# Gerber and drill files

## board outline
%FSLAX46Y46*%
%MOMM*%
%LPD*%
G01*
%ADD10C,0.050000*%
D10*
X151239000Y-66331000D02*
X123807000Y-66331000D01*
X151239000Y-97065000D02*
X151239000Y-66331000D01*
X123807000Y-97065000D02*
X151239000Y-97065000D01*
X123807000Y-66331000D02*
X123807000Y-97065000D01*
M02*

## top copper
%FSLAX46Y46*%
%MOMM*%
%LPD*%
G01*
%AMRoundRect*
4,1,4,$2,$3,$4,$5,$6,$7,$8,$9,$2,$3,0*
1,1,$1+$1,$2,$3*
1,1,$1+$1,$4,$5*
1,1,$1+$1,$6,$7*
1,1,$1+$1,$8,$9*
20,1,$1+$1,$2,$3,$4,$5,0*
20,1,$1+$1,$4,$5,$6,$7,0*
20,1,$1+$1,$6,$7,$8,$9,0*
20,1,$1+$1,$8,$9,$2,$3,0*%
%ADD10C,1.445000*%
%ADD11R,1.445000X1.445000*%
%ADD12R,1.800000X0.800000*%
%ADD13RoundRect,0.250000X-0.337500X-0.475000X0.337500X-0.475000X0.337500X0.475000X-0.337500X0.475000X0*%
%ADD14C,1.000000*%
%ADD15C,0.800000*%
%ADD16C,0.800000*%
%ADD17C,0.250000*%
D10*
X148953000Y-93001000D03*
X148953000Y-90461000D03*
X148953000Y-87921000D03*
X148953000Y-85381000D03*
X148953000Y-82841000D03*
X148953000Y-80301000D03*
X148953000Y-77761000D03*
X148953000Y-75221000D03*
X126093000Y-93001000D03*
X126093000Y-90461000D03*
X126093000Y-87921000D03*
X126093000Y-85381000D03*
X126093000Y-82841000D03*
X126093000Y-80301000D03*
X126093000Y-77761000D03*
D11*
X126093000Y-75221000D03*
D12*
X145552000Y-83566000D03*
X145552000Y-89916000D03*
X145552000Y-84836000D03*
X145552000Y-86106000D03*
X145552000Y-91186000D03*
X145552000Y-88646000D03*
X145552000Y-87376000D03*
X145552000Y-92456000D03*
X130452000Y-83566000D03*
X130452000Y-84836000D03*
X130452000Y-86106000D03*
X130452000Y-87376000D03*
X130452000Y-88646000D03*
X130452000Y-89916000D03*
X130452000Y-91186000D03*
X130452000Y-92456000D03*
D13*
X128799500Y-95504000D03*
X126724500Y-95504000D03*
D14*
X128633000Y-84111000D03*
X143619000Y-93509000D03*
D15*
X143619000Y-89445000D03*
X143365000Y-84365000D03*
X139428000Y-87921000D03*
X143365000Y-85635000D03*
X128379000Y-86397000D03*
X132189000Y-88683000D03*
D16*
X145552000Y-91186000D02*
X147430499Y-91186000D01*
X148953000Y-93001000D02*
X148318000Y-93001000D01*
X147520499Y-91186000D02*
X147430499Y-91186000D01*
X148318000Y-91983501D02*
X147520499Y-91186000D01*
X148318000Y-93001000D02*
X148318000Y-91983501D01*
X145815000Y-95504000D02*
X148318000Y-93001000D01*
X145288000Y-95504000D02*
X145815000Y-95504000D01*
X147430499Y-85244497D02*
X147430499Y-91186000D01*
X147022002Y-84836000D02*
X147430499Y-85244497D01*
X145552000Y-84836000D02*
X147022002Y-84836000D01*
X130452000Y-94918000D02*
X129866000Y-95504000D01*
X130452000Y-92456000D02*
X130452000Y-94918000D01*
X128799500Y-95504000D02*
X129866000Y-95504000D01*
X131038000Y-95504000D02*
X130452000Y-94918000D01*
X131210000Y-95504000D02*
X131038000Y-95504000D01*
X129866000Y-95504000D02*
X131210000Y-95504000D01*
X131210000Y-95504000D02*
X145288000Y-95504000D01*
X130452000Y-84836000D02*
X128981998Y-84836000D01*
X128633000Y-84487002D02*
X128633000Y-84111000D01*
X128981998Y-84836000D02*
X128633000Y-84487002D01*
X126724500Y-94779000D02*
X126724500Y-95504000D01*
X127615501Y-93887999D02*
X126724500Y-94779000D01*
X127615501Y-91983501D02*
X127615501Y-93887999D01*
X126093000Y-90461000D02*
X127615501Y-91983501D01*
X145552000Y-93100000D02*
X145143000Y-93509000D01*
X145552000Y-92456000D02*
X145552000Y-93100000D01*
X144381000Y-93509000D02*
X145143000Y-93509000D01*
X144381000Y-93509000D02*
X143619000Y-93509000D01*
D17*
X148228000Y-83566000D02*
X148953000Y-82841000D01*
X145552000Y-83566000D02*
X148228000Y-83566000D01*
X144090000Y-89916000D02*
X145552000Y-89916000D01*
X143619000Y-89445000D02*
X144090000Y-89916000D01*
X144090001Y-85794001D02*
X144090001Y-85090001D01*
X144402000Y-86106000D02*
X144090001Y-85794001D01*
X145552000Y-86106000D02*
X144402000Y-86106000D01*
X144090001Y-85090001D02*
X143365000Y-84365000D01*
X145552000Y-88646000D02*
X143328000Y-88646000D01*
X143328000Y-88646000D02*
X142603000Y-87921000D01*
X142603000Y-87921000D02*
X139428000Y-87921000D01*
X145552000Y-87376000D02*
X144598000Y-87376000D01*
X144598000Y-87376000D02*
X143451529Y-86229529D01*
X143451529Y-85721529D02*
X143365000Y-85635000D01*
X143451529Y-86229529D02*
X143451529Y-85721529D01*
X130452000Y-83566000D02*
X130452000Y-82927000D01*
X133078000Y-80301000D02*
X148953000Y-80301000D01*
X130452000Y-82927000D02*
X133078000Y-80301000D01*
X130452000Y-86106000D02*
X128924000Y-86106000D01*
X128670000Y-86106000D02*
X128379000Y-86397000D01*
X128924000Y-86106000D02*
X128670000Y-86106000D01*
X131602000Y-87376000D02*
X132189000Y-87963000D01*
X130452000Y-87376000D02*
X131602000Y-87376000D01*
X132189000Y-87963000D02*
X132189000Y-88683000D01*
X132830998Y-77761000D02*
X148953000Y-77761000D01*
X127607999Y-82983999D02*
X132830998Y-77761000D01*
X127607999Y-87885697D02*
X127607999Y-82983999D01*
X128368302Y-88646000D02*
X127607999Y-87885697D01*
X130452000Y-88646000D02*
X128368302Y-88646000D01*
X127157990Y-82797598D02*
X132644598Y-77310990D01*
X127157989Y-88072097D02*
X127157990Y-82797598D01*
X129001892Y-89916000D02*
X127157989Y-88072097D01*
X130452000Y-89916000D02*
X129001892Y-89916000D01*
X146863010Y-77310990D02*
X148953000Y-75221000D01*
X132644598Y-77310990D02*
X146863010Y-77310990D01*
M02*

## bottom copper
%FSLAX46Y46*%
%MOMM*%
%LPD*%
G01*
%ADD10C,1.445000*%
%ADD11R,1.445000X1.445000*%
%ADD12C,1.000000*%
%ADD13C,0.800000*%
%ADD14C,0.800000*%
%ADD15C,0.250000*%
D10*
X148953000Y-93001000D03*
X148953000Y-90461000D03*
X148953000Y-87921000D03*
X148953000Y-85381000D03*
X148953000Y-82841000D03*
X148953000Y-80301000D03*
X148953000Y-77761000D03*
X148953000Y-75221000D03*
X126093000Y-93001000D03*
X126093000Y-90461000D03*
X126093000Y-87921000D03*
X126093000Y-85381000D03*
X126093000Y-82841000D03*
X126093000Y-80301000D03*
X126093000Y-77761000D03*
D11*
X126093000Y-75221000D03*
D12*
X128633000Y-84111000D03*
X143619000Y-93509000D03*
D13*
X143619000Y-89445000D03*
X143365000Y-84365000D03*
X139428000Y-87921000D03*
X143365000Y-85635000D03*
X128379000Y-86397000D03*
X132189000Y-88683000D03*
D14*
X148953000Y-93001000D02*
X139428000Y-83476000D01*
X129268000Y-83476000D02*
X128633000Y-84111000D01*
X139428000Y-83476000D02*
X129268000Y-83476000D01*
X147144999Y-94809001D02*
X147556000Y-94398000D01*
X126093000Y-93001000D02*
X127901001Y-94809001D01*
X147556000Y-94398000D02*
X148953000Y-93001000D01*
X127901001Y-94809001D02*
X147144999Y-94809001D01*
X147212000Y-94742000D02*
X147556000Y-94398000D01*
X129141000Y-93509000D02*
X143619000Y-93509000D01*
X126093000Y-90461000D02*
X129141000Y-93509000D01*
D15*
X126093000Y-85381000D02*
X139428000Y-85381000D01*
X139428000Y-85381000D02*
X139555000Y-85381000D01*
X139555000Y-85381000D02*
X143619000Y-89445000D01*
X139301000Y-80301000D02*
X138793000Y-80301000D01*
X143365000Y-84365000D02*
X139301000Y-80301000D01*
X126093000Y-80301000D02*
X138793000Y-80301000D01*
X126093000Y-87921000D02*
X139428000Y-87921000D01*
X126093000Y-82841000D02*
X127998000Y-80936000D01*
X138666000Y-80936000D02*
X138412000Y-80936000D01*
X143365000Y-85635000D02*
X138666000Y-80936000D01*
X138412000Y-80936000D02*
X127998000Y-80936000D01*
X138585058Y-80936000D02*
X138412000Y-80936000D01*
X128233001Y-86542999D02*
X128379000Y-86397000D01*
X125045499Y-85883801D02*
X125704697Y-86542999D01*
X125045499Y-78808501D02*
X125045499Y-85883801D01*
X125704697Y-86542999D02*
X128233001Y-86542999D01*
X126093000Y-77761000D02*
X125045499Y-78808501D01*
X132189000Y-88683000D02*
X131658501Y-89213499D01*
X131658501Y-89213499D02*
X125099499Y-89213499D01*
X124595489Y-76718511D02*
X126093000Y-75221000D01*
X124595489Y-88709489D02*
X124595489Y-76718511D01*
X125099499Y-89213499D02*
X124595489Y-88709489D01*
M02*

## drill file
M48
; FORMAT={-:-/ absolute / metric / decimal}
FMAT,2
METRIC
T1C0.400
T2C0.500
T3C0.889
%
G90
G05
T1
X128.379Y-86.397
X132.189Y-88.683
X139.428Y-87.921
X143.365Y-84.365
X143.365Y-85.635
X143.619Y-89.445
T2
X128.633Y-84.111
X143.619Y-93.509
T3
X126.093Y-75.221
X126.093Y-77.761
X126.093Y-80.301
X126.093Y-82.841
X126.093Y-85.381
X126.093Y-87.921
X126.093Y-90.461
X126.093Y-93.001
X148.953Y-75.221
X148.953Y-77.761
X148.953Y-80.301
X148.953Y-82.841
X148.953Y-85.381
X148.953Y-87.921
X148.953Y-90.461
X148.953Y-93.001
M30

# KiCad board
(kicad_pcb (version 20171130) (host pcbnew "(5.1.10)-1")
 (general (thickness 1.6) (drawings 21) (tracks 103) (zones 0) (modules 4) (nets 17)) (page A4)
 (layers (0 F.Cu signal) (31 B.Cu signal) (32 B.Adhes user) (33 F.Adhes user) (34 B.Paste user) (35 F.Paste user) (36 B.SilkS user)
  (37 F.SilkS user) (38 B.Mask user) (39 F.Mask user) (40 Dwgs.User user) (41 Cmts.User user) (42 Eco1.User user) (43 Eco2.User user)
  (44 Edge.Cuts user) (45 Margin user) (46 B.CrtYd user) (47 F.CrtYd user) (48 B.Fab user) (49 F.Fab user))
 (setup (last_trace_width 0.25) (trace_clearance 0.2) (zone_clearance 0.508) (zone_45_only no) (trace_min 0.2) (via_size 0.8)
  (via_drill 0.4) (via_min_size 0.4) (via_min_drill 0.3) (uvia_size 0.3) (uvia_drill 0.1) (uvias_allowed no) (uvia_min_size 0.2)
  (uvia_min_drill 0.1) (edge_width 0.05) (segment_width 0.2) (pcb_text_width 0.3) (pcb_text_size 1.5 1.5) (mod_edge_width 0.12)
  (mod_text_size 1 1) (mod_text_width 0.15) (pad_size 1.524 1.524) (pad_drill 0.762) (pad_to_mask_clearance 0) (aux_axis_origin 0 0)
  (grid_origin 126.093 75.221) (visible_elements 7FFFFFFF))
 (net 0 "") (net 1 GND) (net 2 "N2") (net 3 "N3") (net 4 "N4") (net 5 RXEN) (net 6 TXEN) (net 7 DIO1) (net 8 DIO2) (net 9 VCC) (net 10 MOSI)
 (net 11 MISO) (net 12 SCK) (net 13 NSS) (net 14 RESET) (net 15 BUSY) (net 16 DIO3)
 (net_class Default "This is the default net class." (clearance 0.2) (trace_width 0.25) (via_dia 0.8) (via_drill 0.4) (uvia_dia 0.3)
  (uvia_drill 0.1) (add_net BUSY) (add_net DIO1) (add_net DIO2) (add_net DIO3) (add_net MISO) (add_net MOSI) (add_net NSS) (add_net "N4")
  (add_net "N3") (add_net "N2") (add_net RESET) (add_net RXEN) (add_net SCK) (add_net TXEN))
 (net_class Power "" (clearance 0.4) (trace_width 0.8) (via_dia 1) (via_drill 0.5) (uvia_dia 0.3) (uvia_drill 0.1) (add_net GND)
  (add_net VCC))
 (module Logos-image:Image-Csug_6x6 (layer B.Cu) (at 128.379 70.141 180)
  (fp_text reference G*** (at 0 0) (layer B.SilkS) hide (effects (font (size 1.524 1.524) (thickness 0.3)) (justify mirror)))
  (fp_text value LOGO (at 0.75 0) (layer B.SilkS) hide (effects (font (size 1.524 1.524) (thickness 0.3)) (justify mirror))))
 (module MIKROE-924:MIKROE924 (layer F.Cu) (at 126.093 75.221)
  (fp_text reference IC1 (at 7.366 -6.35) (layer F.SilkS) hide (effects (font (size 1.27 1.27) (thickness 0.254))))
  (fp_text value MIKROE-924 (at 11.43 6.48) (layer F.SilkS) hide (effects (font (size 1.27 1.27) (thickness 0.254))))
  (pad 16 thru_hole circle (at 22.86 17.78 90) (size 1.445 1.445) (drill 0.889) (layers *.Cu *.Mask F.SilkS) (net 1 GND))
  (pad 15 thru_hole circle (at 22.86 15.24 90) (size 1.445 1.445) (drill 0.889) (layers *.Cu *.Mask F.SilkS) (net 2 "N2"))
  (pad 14 thru_hole circle (at 22.86 12.7 90) (size 1.445 1.445) (drill 0.889) (layers *.Cu *.Mask F.SilkS) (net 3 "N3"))
  (pad 13 thru_hole circle (at 22.86 10.16 90) (size 1.445 1.445) (drill 0.889) (layers *.Cu *.Mask F.SilkS) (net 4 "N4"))
  (pad 12 thru_hole circle (at 22.86 7.62 90) (size 1.445 1.445) (drill 0.889) (layers *.Cu *.Mask F.SilkS) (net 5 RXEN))
  (pad 11 thru_hole circle (at 22.86 5.08 90) (size 1.445 1.445) (drill 0.889) (layers *.Cu *.Mask F.SilkS) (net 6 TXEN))
  (pad 10 thru_hole circle (at 22.86 2.54 90) (size 1.445 1.445) (drill 0.889) (layers *.Cu *.Mask F.SilkS) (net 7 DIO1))
  (pad 9 thru_hole circle (at 22.86 0 90) (size 1.445 1.445) (drill 0.889) (layers *.Cu *.Mask F.SilkS) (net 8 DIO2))
  (pad 8 thru_hole circle (at 0 17.78 90) (size 1.445 1.445) (drill 0.889) (layers *.Cu *.Mask F.SilkS) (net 1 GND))
  (pad 7 thru_hole circle (at 0 15.24 90) (size 1.445 1.445) (drill 0.889) (layers *.Cu *.Mask F.SilkS) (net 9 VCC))
  (pad 6 thru_hole circle (at 0 12.7 90) (size 1.445 1.445) (drill 0.889) (layers *.Cu *.Mask F.SilkS) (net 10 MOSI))
  (pad 5 thru_hole circle (at 0 10.16 90) (size 1.445 1.445) (drill 0.889) (layers *.Cu *.Mask F.SilkS) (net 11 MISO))
  (pad 4 thru_hole circle (at 0 7.62 90) (size 1.445 1.445) (drill 0.889) (layers *.Cu *.Mask F.SilkS) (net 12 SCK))
  (pad 3 thru_hole circle (at 0 5.08 90) (size 1.445 1.445) (drill 0.889) (layers *.Cu *.Mask F.SilkS) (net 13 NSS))
  (pad 2 thru_hole circle (at 0 2.54 90) (size 1.445 1.445) (drill 0.889) (layers *.Cu *.Mask F.SilkS) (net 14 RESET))
  (pad 1 thru_hole rect (at 0 0 90) (size 1.445 1.445) (drill 0.889) (layers *.Cu *.Mask F.SilkS) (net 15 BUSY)))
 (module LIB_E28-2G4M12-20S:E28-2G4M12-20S (layer F.Cu) (at 135.382 94.996 180)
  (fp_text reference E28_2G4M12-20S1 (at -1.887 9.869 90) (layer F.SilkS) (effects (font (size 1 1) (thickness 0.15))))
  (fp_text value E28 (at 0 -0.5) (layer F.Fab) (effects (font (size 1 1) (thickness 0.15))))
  (pad 8 smd rect (at -10.17 11.43 180) (size 1.8 0.8) (layers F.Cu F.Paste F.Mask) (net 5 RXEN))
  (pad 3 smd rect (at -10.17 5.08 180) (size 1.8 0.8) (layers F.Cu F.Paste F.Mask) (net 11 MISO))
  (pad 7 smd rect (at -10.17 10.16 180) (size 1.8 0.8) (layers F.Cu F.Paste F.Mask) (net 1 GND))
  (pad 6 smd rect (at -10.17 8.89 180) (size 1.8 0.8) (layers F.Cu F.Paste F.Mask) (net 13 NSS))
  (pad 2 smd rect (at -10.17 3.81 180) (size 1.8 0.8) (layers F.Cu F.Paste F.Mask) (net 1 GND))
  (pad 4 smd rect (at -10.17 6.35 180) (size 1.8 0.8) (layers F.Cu F.Paste F.Mask) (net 10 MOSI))
  (pad 5 smd rect (at -10.17 7.62 180) (size 1.8 0.8) (layers F.Cu F.Paste F.Mask) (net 12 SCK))
  (pad 1 smd rect (at -10.17 2.54 180) (size 1.8 0.8) (layers F.Cu F.Paste F.Mask) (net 9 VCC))
  (pad 9 smd rect (at 4.93 11.43 180) (size 1.8 0.8) (layers F.Cu F.Paste F.Mask) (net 6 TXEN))
  (pad 10 smd rect (at 4.93 10.16 180) (size 1.8 0.8) (layers F.Cu F.Paste F.Mask) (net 1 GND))
  (pad 11 smd rect (at 4.93 8.89 180) (size 1.8 0.8) (layers F.Cu F.Paste F.Mask) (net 14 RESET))
  (pad 12 smd rect (at 4.93 7.62 180) (size 1.8 0.8) (layers F.Cu F.Paste F.Mask) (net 15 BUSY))
  (pad 13 smd rect (at 4.93 6.35 180) (size 1.8 0.8) (layers F.Cu F.Paste F.Mask) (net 7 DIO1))
  (pad 14 smd rect (at 4.93 5.08 180) (size 1.8 0.8) (layers F.Cu F.Paste F.Mask) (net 8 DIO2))
  (pad 15 smd rect (at 4.93 3.81 180) (size 1.8 0.8) (layers F.Cu F.Paste F.Mask) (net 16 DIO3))
  (pad 16 smd rect (at 4.93 2.54 180) (size 1.8 0.8) (layers F.Cu F.Paste F.Mask) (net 1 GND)))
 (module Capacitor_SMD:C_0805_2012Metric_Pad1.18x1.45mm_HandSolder (layer F.Cu) (at 127.762 95.504)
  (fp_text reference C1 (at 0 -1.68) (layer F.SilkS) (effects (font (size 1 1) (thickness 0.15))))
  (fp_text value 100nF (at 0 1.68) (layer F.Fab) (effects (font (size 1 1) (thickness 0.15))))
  (pad 2 smd roundrect (at 1.0375 0) (size 1.175 1.45) (layers F.Cu F.Paste F.Mask) (roundrect_rratio 0.2127659574468085) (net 1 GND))
  (pad 1 smd roundrect (at -1.0375 0) (size 1.175 1.45) (layers F.Cu F.Paste F.Mask) (roundrect_rratio 0.2127659574468085) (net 9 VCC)))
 (gr_line (start 151.239 66.331) (end 123.807 66.331) (layer Edge.Cuts) (width 0.05))
 (gr_line (start 151.239 97.065) (end 151.239 66.331) (layer Edge.Cuts) (width 0.05))
 (gr_line (start 123.807 97.065) (end 151.239 97.065) (layer Edge.Cuts) (width 0.05))
 (gr_line (start 123.807 66.331) (end 123.807 97.065) (layer Edge.Cuts) (width 0.05))
 (segment (start 145.552 91.186) (end 147.430499 91.186) (width 0.8) (layer F.Cu) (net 1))
 (segment (start 148.953 93.001) (end 148.318 93.001) (width 0.8) (layer F.Cu) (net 1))
 (segment (start 147.520499 91.186) (end 147.430499 91.186) (width 0.8) (layer F.Cu) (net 1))
 (segment (start 148.318 91.983501) (end 147.520499 91.186) (width 0.8) (layer F.Cu) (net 1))
 (segment (start 148.318 93.001) (end 148.318 91.983501) (width 0.8) (layer F.Cu) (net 1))
 (segment (start 145.815 95.504) (end 148.318 93.001) (width 0.8) (layer F.Cu) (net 1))
 (segment (start 145.288 95.504) (end 145.815 95.504) (width 0.8) (layer F.Cu) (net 1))
 (segment (start 147.430499 85.244497) (end 147.430499 91.186) (width 0.8) (layer F.Cu) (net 1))
 (segment (start 147.022002 84.836) (end 147.430499 85.244497) (width 0.8) (layer F.Cu) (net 1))
 (segment (start 145.552 84.836) (end 147.022002 84.836) (width 0.8) (layer F.Cu) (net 1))
 (segment (start 130.452 94.918) (end 129.866 95.504) (width 0.8) (layer F.Cu) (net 1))
 (segment (start 130.452 92.456) (end 130.452 94.918) (width 0.8) (layer F.Cu) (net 1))
 (segment (start 128.7995 95.504) (end 129.866 95.504) (width 0.8) (layer F.Cu) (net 1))
 (segment (start 131.038 95.504) (end 130.452 94.918) (width 0.8) (layer F.Cu) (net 1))
 (segment (start 131.21 95.504) (end 131.038 95.504) (width 0.8) (layer F.Cu) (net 1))
 (segment (start 129.866 95.504) (end 131.21 95.504) (width 0.8) (layer F.Cu) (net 1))
 (segment (start 131.21 95.504) (end 145.288 95.504) (width 0.8) (layer F.Cu) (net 1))
 (via (at 128.633 84.111) (size 1) (drill 0.5) (layers F.Cu B.Cu) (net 1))
 (segment (start 130.452 84.836) (end 128.981998 84.836) (width 0.8) (layer F.Cu) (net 1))
 (segment (start 148.953 93.001) (end 139.428 83.476) (width 0.8) (layer B.Cu) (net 1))
 (segment (start 128.633 84.487002) (end 128.633 84.111) (width 0.8) (layer F.Cu) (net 1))
 (segment (start 128.981998 84.836) (end 128.633 84.487002) (width 0.8) (layer F.Cu) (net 1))
 (segment (start 129.268 83.476) (end 128.633 84.111) (width 0.8) (layer B.Cu) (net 1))
 (segment (start 139.428 83.476) (end 129.268 83.476) (width 0.8) (layer B.Cu) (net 1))
 (segment (start 147.144999 94.809001) (end 147.556 94.398) (width 0.8) (layer B.Cu) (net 1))
 (segment (start 126.093 93.001) (end 127.901001 94.809001) (width 0.8) (layer B.Cu) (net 1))
 (segment (start 147.556 94.398) (end 148.953 93.001) (width 0.8) (layer B.Cu) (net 1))
 (segment (start 127.901001 94.809001) (end 147.144999 94.809001) (width 0.8) (layer B.Cu) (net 1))
 (segment (start 147.212 94.742) (end 147.556 94.398) (width 0.8) (layer B.Cu) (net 1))
 (segment (start 126.7245 94.779) (end 126.7245 95.504) (width 0.8) (layer F.Cu) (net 9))
 (segment (start 127.615501 93.887999) (end 126.7245 94.779) (width 0.8) (layer F.Cu) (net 9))
 (segment (start 127.615501 91.983501) (end 127.615501 93.887999) (width 0.8) (layer F.Cu) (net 9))
 (segment (start 126.093 90.461) (end 127.615501 91.983501) (width 0.8) (layer F.Cu) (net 9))
 (via (at 143.619 93.509) (size 1) (drill 0.5) (layers F.Cu B.Cu) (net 9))
 (segment (start 145.552 93.1) (end 145.143 93.509) (width 0.8) (layer F.Cu) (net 9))
 (segment (start 145.552 92.456) (end 145.552 93.1) (width 0.8) (layer F.Cu) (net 9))
 (segment (start 144.381 93.509) (end 145.143 93.509) (width 0.8) (layer F.Cu) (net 9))
 (segment (start 144.381 93.509) (end 143.619 93.509) (width 0.8) (layer F.Cu) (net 9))
 (segment (start 129.141 93.509) (end 143.619 93.509) (width 0.8) (layer B.Cu) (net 9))
 (segment (start 126.093 90.461) (end 129.141 93.509) (width 0.8) (layer B.Cu) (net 9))
 (segment (start 148.228 83.566) (end 148.953 82.841) (width 0.25) (layer F.Cu) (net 5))
 (segment (start 145.552 83.566) (end 148.228 83.566) (width 0.25) (layer F.Cu) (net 5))
 (segment (start 126.093 85.381) (end 139.428 85.381) (width 0.25) (layer B.Cu) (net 11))
 (segment (start 139.428 85.381) (end 139.555 85.381) (width 0.25) (layer B.Cu) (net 11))
 (via (at 143.619 89.445) (size 0.8) (drill 0.4) (layers F.Cu B.Cu) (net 11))
 (segment (start 139.555 85.381) (end 143.619 89.445) (width 0.25) (layer B.Cu) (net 11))
 (segment (start 144.09 89.916) (end 145.552 89.916) (width 0.25) (layer F.Cu) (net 11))
 (segment (start 143.619 89.445) (end 144.09 89.916) (width 0.25) (layer F.Cu) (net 11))
 (segment (start 144.090001 85.794001) (end 144.090001 85.090001) (width 0.25) (layer F.Cu) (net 13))
 (segment (start 144.402 86.106) (end 144.090001 85.794001) (width 0.25) (layer F.Cu) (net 13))
 (segment (start 145.552 86.106) (end 144.402 86.106) (width 0.25) (layer F.Cu) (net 13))
 (segment (start 144.090001 85.090001) (end 143.365 84.365) (width 0.25) (layer F.Cu) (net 13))
 (via (at 143.365 84.365) (size 0.8) (drill 0.4) (layers F.Cu B.Cu) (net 13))
 (segment (start 139.301 80.301) (end 138.793 80.301) (width 0.25) (layer B.Cu) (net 13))
 (segment (start 143.365 84.365) (end 139.301 80.301) (width 0.25) (layer B.Cu) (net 13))
 (segment (start 126.093 80.301) (end 138.793 80.301) (width 0.25) (layer B.Cu) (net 13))
 (segment (start 126.093 87.921) (end 139.428 87.921) (width 0.25) (layer B.Cu) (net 10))
 (via (at 139.428 87.921) (size 0.8) (drill 0.4) (layers F.Cu B.Cu) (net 10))
 (segment (start 145.552 88.646) (end 143.328 88.646) (width 0.25) (layer F.Cu) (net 10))
 (segment (start 143.328 88.646) (end 142.603 87.921) (width 0.25) (layer F.Cu) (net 10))
 (segment (start 142.603 87.921) (end 139.428 87.921) (width 0.25) (layer F.Cu) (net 10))
 (segment (start 126.093 82.841) (end 127.998 80.936) (width 0.25) (layer B.Cu) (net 12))
 (segment (start 145.552 87.376) (end 144.598 87.376) (width 0.25) (layer F.Cu) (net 12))
 (segment (start 144.598 87.376) (end 143.451529 86.229529) (width 0.25) (layer F.Cu) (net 12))
 (via (at 143.365 85.635) (size 0.8) (drill 0.4) (layers F.Cu B.Cu) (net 12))
 (segment (start 143.451529 85.721529) (end 143.365 85.635) (width 0.25) (layer F.Cu) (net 12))
 (segment (start 143.451529 86.229529) (end 143.451529 85.721529) (width 0.25) (layer F.Cu) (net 12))
 (segment (start 138.666 80.936) (end 138.412 80.936) (width 0.25) (layer B.Cu) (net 12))
 (segment (start 143.365 85.635) (end 138.666 80.936) (width 0.25) (layer B.Cu) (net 12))
 (segment (start 138.412 80.936) (end 127.998 80.936) (width 0.25) (layer B.Cu) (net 12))
 (segment (start 138.585058 80.936) (end 138.412 80.936) (width 0.25) (layer B.Cu) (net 12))
 (segment (start 130.452 83.566) (end 130.452 82.927) (width 0.25) (layer F.Cu) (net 6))
 (segment (start 133.078 80.301) (end 148.953 80.301) (width 0.25) (layer F.Cu) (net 6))
 (segment (start 130.452 82.927) (end 133.078 80.301) (width 0.25) (layer F.Cu) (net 6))
 (via (at 128.379 86.397) (size 0.8) (drill 0.4) (layers F.Cu B.Cu) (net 14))
 (segment (start 130.452 86.106) (end 128.924 86.106) (width 0.25) (layer F.Cu) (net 14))
 (segment (start 128.67 86.106) (end 128.379 86.397) (width 0.25) (layer F.Cu) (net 14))
 (segment (start 128.924 86.106) (end 128.67 86.106) (width 0.25) (layer F.Cu) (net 14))
 (segment (start 128.233001 86.542999) (end 128.379 86.397) (width 0.25) (layer B.Cu) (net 14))
 (segment (start 125.045499 85.883801) (end 125.704697 86.542999) (width 0.25) (layer B.Cu) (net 14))
 (segment (start 125.045499 78.808501) (end 125.045499 85.883801) (width 0.25) (layer B.Cu) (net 14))
 (segment (start 125.704697 86.542999) (end 128.233001 86.542999) (width 0.25) (layer B.Cu) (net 14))
 (segment (start 126.093 77.761) (end 125.045499 78.808501) (width 0.25) (layer B.Cu) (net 14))
 (segment (start 131.602 87.376) (end 132.189 87.963) (width 0.25) (layer F.Cu) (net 15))
 (segment (start 130.452 87.376) (end 131.602 87.376) (width 0.25) (layer F.Cu) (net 15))
 (via (at 132.189 88.683) (size 0.8) (drill 0.4) (layers F.Cu B.Cu) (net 15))
 (segment (start 132.189 87.963) (end 132.189 88.683) (width 0.25) (layer F.Cu) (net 15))
 (segment (start 132.189 88.683) (end 131.658501 89.213499) (width 0.25) (layer B.Cu) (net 15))
 (segment (start 131.658501 89.213499) (end 125.099499 89.213499) (width 0.25) (layer B.Cu) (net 15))
 (segment (start 124.595489 76.718511) (end 126.093 75.221) (width 0.25) (layer B.Cu) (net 15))
 (segment (start 124.595489 88.709489) (end 124.595489 76.718511) (width 0.25) (layer B.Cu) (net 15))
 (segment (start 125.099499 89.213499) (end 124.595489 88.709489) (width 0.25) (layer B.Cu) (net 15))
 (segment (start 132.830998 77.761) (end 148.953 77.761) (width 0.25) (layer F.Cu) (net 7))
 (segment (start 127.607999 82.983999) (end 132.830998 77.761) (width 0.25) (layer F.Cu) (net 7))
 (segment (start 127.607999 87.885697) (end 127.607999 82.983999) (width 0.25) (layer F.Cu) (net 7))
 (segment (start 128.368302 88.646) (end 127.607999 87.885697) (width 0.25) (layer F.Cu) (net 7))
 (segment (start 130.452 88.646) (end 128.368302 88.646) (width 0.25) (layer F.Cu) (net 7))
 (segment (start 127.15799 82.797598) (end 132.644598 77.31099) (width 0.25) (layer F.Cu) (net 8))
 (segment (start 127.157989 88.072097) (end 127.15799 82.797598) (width 0.25) (layer F.Cu) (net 8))
 (segment (start 129.001892 89.916) (end 127.157989 88.072097) (width 0.25) (layer F.Cu) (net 8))
 (segment (start 130.452 89.916) (end 129.001892 89.916) (width 0.25) (layer F.Cu) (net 8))
 (segment (start 146.86301 77.31099) (end 148.953 75.221) (width 0.25) (layer F.Cu) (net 8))
 (segment (start 132.644598 77.31099) (end 146.86301 77.31099) (width 0.25) (layer F.Cu) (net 8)))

